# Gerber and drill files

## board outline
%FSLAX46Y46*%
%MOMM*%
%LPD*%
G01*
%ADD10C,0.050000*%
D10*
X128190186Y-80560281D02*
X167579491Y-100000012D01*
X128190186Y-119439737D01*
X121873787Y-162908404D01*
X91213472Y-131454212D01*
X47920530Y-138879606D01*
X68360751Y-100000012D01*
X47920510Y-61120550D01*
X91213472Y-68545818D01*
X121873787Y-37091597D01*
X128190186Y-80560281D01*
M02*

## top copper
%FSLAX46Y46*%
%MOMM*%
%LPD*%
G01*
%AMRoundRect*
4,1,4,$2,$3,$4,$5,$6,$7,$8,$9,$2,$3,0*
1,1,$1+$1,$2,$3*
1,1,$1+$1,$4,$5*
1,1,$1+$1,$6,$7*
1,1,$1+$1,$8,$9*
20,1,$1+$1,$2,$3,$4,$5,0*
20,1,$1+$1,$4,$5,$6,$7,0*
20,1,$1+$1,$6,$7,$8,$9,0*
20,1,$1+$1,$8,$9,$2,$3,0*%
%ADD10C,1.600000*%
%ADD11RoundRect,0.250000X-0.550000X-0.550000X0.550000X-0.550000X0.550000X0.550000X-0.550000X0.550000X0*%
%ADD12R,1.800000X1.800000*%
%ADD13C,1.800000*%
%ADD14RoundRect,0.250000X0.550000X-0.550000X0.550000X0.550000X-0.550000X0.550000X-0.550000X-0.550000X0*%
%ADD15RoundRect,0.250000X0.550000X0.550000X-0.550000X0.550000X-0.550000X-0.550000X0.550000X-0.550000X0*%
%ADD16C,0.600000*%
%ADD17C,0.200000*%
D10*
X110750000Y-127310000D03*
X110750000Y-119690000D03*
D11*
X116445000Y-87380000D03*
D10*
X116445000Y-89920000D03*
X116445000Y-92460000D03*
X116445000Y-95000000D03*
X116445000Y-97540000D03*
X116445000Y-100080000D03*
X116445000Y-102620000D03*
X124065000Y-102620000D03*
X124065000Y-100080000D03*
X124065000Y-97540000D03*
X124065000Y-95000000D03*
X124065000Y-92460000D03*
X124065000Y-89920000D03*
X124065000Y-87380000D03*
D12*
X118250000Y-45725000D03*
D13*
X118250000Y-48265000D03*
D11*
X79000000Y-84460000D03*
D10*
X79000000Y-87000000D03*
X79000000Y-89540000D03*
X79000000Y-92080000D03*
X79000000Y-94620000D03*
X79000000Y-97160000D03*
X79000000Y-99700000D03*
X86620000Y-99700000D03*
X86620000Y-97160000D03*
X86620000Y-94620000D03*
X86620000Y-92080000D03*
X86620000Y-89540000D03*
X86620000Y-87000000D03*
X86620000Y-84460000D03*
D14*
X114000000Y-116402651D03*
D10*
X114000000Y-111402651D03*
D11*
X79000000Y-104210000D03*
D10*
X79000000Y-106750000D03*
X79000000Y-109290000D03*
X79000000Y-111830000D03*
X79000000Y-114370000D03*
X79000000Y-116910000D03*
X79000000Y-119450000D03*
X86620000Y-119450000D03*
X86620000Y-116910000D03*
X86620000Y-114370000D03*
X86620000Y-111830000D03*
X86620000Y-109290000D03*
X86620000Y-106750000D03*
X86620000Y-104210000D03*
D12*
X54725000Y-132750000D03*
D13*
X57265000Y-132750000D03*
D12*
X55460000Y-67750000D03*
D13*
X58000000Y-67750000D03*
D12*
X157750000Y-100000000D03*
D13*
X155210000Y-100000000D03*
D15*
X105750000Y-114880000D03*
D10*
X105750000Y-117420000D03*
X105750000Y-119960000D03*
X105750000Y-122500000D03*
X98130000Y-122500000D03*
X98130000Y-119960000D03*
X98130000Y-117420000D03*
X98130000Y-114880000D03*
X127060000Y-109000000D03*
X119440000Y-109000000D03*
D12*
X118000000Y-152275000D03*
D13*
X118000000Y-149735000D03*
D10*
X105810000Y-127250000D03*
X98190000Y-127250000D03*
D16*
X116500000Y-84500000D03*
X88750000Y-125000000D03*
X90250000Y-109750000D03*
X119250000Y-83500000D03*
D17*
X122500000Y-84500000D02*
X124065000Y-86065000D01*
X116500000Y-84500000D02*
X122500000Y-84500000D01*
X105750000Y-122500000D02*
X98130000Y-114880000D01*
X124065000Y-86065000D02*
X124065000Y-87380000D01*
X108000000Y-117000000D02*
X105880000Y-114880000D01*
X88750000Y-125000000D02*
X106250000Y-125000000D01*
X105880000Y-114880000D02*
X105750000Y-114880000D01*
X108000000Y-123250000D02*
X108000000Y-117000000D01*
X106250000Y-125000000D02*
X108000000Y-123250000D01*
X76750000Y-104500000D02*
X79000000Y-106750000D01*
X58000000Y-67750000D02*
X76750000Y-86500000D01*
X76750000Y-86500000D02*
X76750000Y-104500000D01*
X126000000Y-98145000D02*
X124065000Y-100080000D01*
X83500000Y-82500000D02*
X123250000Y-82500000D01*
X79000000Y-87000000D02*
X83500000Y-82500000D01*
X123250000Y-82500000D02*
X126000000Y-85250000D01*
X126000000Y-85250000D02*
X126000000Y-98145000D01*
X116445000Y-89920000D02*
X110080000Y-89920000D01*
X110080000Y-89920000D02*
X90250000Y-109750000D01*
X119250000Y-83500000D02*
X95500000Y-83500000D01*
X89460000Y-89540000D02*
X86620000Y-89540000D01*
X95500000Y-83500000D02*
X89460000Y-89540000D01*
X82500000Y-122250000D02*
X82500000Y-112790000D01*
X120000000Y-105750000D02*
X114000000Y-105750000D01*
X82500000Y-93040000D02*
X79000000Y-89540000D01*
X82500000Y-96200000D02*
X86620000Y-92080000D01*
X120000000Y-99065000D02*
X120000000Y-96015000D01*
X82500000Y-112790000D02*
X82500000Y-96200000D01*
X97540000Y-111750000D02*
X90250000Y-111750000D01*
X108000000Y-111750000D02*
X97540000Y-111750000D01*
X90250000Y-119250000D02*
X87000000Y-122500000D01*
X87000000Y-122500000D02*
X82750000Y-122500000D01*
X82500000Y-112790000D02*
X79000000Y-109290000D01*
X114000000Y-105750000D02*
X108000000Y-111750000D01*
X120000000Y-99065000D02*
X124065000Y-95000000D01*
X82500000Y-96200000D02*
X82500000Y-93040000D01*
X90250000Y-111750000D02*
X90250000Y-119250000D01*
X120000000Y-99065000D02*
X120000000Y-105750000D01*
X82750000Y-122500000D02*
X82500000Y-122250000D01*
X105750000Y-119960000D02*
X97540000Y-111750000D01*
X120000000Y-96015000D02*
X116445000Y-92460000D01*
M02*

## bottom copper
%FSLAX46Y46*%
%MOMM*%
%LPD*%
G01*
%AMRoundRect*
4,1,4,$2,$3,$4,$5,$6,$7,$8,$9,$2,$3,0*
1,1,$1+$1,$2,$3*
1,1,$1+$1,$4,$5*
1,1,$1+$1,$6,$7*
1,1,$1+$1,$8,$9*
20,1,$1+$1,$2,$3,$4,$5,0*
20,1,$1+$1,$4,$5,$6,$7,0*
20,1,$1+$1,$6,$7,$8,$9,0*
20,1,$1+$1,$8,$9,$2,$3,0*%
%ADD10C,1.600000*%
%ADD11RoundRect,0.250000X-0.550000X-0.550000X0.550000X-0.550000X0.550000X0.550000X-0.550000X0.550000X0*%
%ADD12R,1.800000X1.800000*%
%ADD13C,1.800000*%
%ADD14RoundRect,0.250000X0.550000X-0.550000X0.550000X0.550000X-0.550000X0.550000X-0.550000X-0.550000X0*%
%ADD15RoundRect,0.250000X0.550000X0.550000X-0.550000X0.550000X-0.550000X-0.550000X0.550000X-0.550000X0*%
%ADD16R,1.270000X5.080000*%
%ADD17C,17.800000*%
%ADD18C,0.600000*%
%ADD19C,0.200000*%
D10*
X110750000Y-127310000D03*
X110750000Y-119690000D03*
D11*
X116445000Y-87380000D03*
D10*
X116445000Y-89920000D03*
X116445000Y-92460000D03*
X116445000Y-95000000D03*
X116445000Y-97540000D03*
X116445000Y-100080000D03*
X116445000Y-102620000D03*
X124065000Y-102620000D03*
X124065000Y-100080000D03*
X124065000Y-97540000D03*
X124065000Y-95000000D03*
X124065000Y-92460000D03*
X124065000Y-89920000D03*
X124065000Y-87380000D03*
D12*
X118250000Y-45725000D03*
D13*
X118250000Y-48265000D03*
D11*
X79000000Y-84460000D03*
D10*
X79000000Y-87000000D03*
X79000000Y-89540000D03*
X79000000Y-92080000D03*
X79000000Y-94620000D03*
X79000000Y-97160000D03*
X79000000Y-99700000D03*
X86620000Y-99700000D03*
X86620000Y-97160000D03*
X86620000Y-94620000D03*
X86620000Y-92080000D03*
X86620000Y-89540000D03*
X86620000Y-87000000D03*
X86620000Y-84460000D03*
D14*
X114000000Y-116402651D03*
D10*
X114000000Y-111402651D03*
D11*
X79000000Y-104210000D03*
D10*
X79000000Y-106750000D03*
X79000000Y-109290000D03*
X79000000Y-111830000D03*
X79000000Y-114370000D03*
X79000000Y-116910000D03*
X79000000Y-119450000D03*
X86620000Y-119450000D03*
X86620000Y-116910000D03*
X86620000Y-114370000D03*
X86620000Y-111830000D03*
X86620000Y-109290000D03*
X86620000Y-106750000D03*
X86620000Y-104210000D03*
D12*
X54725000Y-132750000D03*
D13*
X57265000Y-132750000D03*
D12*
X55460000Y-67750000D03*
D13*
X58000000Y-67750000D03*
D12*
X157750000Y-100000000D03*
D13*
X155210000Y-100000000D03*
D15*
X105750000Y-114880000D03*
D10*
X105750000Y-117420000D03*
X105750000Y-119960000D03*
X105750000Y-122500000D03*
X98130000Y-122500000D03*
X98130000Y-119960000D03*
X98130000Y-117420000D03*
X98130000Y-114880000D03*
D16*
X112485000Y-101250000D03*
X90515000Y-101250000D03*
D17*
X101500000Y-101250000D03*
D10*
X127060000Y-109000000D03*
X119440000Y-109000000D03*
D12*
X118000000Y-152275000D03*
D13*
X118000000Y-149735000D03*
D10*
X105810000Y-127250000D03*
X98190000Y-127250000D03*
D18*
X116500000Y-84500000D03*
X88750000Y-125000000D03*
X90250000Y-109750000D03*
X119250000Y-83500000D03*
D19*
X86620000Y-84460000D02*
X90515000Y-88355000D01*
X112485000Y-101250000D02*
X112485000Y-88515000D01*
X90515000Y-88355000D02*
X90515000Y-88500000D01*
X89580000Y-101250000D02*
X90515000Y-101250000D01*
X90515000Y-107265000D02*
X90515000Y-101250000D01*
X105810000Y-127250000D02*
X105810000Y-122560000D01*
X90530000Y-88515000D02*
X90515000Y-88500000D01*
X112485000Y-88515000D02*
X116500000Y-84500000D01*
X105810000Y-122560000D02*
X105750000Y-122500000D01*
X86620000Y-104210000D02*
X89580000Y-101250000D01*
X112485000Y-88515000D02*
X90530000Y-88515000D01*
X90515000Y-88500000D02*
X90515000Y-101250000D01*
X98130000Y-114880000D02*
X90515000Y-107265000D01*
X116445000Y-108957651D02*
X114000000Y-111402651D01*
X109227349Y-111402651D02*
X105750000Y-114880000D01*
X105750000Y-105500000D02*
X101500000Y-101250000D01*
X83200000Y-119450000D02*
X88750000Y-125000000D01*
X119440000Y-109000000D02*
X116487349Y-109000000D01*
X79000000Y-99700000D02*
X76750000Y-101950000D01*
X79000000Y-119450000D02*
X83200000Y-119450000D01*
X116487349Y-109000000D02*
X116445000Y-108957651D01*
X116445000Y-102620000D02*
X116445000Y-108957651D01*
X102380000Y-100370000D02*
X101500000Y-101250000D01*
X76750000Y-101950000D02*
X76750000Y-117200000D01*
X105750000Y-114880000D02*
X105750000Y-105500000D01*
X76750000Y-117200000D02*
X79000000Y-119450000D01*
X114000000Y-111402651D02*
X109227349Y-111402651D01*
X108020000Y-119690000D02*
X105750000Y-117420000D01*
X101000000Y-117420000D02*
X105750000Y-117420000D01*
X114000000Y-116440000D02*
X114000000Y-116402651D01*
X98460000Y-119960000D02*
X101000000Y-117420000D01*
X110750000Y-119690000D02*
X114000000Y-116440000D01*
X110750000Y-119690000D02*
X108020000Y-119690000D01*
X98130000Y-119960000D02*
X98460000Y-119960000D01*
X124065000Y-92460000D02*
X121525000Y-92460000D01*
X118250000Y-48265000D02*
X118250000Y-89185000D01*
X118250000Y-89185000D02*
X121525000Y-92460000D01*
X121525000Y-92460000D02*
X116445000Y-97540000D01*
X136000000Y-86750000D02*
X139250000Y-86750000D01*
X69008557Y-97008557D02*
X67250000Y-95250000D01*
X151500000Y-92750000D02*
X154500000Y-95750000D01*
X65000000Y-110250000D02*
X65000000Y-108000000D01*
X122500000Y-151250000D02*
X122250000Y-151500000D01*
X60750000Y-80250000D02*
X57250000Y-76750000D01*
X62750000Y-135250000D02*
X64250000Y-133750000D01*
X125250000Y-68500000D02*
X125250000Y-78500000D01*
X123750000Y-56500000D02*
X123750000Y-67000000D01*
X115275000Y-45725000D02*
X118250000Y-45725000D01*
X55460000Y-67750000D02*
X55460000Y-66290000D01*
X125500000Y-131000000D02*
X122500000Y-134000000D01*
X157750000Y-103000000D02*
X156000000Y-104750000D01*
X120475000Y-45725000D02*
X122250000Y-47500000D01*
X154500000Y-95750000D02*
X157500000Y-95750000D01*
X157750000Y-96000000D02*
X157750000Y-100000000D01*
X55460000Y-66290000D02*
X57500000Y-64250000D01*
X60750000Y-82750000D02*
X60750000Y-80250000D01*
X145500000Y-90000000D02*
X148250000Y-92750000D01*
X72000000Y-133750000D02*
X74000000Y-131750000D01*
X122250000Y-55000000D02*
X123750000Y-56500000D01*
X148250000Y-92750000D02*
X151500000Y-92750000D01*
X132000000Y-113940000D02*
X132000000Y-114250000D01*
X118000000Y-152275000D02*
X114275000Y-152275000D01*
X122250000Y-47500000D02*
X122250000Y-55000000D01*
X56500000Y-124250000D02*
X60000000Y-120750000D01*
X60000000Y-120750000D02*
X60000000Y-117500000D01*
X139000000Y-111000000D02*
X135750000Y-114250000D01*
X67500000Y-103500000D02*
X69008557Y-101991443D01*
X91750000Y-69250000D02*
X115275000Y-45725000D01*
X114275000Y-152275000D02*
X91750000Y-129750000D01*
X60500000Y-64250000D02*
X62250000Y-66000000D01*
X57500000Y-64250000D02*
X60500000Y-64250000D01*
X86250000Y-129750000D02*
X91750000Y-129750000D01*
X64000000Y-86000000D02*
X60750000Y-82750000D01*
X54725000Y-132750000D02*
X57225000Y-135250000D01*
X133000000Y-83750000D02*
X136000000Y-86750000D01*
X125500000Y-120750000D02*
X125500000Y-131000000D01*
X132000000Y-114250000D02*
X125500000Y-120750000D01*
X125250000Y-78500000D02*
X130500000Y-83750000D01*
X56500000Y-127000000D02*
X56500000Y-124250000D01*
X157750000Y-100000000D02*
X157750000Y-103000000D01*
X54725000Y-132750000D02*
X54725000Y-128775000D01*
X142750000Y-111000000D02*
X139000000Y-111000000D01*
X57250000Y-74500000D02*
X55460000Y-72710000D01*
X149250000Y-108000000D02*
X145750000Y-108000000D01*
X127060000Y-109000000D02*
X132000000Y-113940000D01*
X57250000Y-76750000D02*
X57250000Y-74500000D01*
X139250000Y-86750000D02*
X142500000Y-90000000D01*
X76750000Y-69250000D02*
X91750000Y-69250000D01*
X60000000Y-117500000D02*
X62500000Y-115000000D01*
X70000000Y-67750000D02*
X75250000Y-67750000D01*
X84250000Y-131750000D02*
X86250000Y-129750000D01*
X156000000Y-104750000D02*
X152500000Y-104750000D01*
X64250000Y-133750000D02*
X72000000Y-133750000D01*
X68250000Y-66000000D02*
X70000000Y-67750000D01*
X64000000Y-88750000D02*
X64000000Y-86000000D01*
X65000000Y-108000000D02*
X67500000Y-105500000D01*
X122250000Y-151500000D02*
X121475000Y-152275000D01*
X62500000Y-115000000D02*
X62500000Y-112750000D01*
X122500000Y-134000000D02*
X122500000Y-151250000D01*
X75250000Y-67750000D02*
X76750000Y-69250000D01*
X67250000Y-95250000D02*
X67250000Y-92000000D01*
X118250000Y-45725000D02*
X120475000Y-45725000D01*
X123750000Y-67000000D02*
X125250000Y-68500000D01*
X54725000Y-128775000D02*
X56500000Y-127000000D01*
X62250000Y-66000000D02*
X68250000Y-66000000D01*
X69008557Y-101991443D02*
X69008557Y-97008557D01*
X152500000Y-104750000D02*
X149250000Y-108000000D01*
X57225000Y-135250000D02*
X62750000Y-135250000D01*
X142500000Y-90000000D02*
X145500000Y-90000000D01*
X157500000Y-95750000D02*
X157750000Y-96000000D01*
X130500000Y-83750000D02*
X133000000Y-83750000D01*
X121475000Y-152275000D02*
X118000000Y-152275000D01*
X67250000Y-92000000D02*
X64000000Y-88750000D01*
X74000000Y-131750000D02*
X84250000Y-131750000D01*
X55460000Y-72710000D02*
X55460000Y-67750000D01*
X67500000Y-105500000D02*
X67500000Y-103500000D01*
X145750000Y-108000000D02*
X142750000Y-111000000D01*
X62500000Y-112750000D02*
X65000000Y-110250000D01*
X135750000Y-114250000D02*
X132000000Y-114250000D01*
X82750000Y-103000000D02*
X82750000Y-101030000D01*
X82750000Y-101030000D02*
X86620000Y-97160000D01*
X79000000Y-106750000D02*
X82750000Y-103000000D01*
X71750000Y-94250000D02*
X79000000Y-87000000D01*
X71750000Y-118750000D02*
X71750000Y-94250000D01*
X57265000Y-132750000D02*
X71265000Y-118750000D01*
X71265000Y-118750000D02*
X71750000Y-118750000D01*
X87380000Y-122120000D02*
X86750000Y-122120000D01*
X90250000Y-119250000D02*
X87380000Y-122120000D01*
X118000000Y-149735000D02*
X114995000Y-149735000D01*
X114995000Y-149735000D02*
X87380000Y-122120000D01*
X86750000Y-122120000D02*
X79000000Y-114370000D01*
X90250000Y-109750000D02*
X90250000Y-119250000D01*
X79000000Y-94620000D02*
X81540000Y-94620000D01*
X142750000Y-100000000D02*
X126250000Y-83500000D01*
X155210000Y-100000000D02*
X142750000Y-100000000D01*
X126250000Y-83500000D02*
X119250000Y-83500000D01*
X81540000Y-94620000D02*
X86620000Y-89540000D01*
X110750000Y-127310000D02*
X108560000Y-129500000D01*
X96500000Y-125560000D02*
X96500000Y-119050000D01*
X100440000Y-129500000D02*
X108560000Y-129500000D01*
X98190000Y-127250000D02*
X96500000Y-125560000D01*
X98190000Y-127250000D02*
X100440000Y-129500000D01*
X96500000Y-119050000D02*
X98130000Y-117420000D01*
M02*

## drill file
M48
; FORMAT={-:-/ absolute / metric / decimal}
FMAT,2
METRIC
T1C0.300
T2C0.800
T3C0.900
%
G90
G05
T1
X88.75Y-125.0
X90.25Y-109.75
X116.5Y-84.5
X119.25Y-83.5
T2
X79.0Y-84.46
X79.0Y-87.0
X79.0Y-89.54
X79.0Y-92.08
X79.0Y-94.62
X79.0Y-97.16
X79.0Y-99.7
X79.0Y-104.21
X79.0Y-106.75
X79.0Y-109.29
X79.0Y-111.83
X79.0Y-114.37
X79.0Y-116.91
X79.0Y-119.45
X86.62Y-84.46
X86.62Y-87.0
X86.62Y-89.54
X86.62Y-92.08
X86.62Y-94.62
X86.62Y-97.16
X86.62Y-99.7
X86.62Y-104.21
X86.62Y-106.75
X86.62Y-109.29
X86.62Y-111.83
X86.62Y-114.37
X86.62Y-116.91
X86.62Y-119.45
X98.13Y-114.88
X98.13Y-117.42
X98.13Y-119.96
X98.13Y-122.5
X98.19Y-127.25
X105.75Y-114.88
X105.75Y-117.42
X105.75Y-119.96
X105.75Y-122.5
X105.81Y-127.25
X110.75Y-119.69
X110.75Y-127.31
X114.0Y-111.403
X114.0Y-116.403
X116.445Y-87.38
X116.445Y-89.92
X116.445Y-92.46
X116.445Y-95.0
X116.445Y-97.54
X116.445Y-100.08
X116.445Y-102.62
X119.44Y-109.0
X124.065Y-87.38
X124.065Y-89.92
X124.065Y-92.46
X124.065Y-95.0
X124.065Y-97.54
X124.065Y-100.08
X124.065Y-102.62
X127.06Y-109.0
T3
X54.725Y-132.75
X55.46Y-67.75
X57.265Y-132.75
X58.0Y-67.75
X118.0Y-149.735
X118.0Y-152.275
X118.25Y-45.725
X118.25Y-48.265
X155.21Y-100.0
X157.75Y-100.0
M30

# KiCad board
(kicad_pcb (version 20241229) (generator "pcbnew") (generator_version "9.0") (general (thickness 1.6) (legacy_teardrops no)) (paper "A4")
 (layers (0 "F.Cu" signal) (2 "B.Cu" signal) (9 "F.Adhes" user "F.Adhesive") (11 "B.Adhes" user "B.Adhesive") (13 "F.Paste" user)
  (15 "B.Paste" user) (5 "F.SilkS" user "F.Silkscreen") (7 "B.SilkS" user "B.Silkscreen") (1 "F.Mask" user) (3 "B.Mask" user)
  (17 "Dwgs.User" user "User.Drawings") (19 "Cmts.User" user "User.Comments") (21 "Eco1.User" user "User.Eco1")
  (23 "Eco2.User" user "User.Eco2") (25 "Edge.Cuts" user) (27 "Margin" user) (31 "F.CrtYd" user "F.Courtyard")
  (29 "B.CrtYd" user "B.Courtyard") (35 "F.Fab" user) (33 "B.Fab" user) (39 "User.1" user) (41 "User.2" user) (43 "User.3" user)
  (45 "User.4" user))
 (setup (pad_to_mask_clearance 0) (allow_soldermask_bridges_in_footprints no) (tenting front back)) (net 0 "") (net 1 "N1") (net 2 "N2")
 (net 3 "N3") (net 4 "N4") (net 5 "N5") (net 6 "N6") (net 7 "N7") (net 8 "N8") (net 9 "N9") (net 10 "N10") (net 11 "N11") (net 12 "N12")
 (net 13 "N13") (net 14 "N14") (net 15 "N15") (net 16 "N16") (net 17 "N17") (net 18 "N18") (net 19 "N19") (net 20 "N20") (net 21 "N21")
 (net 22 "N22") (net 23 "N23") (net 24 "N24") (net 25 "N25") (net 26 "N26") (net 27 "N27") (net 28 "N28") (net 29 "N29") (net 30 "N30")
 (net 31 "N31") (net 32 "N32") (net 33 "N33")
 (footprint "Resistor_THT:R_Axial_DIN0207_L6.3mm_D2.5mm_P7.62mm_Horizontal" (layer "F.Cu") (at 110.75 127.31 90)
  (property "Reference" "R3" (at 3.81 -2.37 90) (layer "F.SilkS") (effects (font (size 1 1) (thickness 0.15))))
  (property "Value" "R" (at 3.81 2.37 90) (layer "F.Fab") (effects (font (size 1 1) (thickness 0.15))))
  (pad "1" thru_hole circle (at 0 0 90) (size 1.6 1.6) (drill 0.8) (layers "*.Cu" "*.Mask") (remove_unused_layers no) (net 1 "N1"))
  (pad "2" thru_hole circle (at 7.62 0 90) (size 1.6 1.6) (drill 0.8) (layers "*.Cu" "*.Mask") (remove_unused_layers no) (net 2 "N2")))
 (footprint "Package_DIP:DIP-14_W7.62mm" (layer "F.Cu") (at 116.445 87.38)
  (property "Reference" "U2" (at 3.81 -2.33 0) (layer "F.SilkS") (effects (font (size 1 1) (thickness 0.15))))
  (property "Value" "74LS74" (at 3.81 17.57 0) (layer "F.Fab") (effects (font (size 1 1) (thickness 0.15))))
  (pad "1" thru_hole roundrect (at 0 0) (size 1.6 1.6) (drill 0.8) (layers "*.Cu" "*.Mask") (remove_unused_layers no)
   (roundrect_rratio 0.15625) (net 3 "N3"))
  (pad "2" thru_hole circle (at 0 2.54) (size 1.6 1.6) (drill 0.8) (layers "*.Cu" "*.Mask") (remove_unused_layers no) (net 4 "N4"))
  (pad "3" thru_hole circle (at 0 5.08) (size 1.6 1.6) (drill 0.8) (layers "*.Cu" "*.Mask") (remove_unused_layers no) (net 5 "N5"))
  (pad "4" thru_hole circle (at 0 7.62) (size 1.6 1.6) (drill 0.8) (layers "*.Cu" "*.Mask") (remove_unused_layers no) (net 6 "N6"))
  (pad "5" thru_hole circle (at 0 10.16) (size 1.6 1.6) (drill 0.8) (layers "*.Cu" "*.Mask") (remove_unused_layers no) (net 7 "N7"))
  (pad "6" thru_hole circle (at 0 12.7) (size 1.6 1.6) (drill 0.8) (layers "*.Cu" "*.Mask") (remove_unused_layers no) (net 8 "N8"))
  (pad "7" thru_hole circle (at 0 15.24) (size 1.6 1.6) (drill 0.8) (layers "*.Cu" "*.Mask") (remove_unused_layers no) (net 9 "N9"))
  (pad "8" thru_hole circle (at 7.62 15.24) (size 1.6 1.6) (drill 0.8) (layers "*.Cu" "*.Mask") (remove_unused_layers no) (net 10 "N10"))
  (pad "9" thru_hole circle (at 7.62 12.7) (size 1.6 1.6) (drill 0.8) (layers "*.Cu" "*.Mask") (remove_unused_layers no) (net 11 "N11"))
  (pad "10" thru_hole circle (at 7.62 10.16) (size 1.6 1.6) (drill 0.8) (layers "*.Cu" "*.Mask") (remove_unused_layers no) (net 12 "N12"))
  (pad "11" thru_hole circle (at 7.62 7.62) (size 1.6 1.6) (drill 0.8) (layers "*.Cu" "*.Mask") (remove_unused_layers no) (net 5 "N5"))
  (pad "12" thru_hole circle (at 7.62 5.08) (size 1.6 1.6) (drill 0.8) (layers "*.Cu" "*.Mask") (remove_unused_layers no) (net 7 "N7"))
  (pad "13" thru_hole circle (at 7.62 2.54) (size 1.6 1.6) (drill 0.8) (layers "*.Cu" "*.Mask") (remove_unused_layers no) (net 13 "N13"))
  (pad "14" thru_hole circle (at 7.62 0) (size 1.6 1.6) (drill 0.8) (layers "*.Cu" "*.Mask") (remove_unused_layers no) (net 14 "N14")))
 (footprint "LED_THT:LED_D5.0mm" (layer "F.Cu") (at 118.25 45.725 -90)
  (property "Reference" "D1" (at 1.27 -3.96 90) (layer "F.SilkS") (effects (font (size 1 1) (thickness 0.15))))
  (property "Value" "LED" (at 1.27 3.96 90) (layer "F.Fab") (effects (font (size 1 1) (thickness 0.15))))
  (pad "1" thru_hole rect (at 0 0 270) (size 1.8 1.8) (drill 0.9) (layers "*.Cu" "*.Mask") (remove_unused_layers no) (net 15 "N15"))
  (pad "2" thru_hole circle (at 2.54 0 270) (size 1.8 1.8) (drill 0.9) (layers "*.Cu" "*.Mask") (remove_unused_layers no) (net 7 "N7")))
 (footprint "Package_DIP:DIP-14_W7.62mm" (layer "F.Cu") (at 79 84.46)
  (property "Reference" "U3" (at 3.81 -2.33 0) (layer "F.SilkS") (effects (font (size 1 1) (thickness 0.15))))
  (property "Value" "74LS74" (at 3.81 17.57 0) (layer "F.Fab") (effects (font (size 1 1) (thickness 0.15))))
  (pad "1" thru_hole roundrect (at 0 0) (size 1.6 1.6) (drill 0.8) (layers "*.Cu" "*.Mask") (remove_unused_layers no)
   (roundrect_rratio 0.15625) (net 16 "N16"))
  (pad "2" thru_hole circle (at 0 2.54) (size 1.6 1.6) (drill 0.8) (layers "*.Cu" "*.Mask") (remove_unused_layers no) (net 11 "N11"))
  (pad "3" thru_hole circle (at 0 5.08) (size 1.6 1.6) (drill 0.8) (layers "*.Cu" "*.Mask") (remove_unused_layers no) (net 5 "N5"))
  (pad "4" thru_hole circle (at 0 7.62) (size 1.6 1.6) (drill 0.8) (layers "*.Cu" "*.Mask") (remove_unused_layers no) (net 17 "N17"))
  (pad "5" thru_hole circle (at 0 10.16) (size 1.6 1.6) (drill 0.8) (layers "*.Cu" "*.Mask") (remove_unused_layers no) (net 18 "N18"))
  (pad "6" thru_hole circle (at 0 12.7) (size 1.6 1.6) (drill 0.8) (layers "*.Cu" "*.Mask") (remove_unused_layers no) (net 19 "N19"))
  (pad "7" thru_hole circle (at 0 15.24) (size 1.6 1.6) (drill 0.8) (layers "*.Cu" "*.Mask") (remove_unused_layers no) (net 9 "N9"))
  (pad "8" thru_hole circle (at 7.62 15.24) (size 1.6 1.6) (drill 0.8) (layers "*.Cu" "*.Mask") (remove_unused_layers no) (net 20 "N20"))
  (pad "9" thru_hole circle (at 7.62 12.7) (size 1.6 1.6) (drill 0.8) (layers "*.Cu" "*.Mask") (remove_unused_layers no) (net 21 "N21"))
  (pad "10" thru_hole circle (at 7.62 10.16) (size 1.6 1.6) (drill 0.8) (layers "*.Cu" "*.Mask") (remove_unused_layers no) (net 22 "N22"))
  (pad "11" thru_hole circle (at 7.62 7.62) (size 1.6 1.6) (drill 0.8) (layers "*.Cu" "*.Mask") (remove_unused_layers no) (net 5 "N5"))
  (pad "12" thru_hole circle (at 7.62 5.08) (size 1.6 1.6) (drill 0.8) (layers "*.Cu" "*.Mask") (remove_unused_layers no) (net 18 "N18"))
  (pad "13" thru_hole circle (at 7.62 2.54) (size 1.6 1.6) (drill 0.8) (layers "*.Cu" "*.Mask") (remove_unused_layers no) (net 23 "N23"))
  (pad "14" thru_hole circle (at 7.62 0) (size 1.6 1.6) (drill 0.8) (layers "*.Cu" "*.Mask") (remove_unused_layers no) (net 14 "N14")))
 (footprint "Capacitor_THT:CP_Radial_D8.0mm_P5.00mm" (layer "F.Cu") (at 114 116.402651 90)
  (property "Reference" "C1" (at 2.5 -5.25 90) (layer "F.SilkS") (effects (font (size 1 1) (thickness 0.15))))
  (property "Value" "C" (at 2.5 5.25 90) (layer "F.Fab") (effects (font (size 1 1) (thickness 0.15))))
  (pad "1" thru_hole roundrect (at 0 0 90) (size 1.6 1.6) (drill 0.8) (layers "*.Cu" "*.Mask") (remove_unused_layers no)
   (roundrect_rratio 0.15625) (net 2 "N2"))
  (pad "2" thru_hole circle (at 5 0 90) (size 1.6 1.6) (drill 0.8) (layers "*.Cu" "*.Mask") (remove_unused_layers no) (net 9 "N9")))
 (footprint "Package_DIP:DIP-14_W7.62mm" (layer "F.Cu") (at 79 104.21)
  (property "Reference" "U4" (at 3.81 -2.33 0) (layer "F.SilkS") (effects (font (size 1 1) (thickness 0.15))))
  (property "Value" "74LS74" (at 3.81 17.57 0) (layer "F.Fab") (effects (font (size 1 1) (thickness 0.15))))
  (pad "1" thru_hole roundrect (at 0 0) (size 1.6 1.6) (drill 0.8) (layers "*.Cu" "*.Mask") (remove_unused_layers no)
   (roundrect_rratio 0.15625) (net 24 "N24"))
  (pad "2" thru_hole circle (at 0 2.54) (size 1.6 1.6) (drill 0.8) (layers "*.Cu" "*.Mask") (remove_unused_layers no) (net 21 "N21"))
  (pad "3" thru_hole circle (at 0 5.08) (size 1.6 1.6) (drill 0.8) (layers "*.Cu" "*.Mask") (remove_unused_layers no) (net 5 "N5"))
  (pad "4" thru_hole circle (at 0 7.62) (size 1.6 1.6) (drill 0.8) (layers "*.Cu" "*.Mask") (remove_unused_layers no) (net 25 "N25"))
  (pad "5" thru_hole circle (at 0 10.16) (size 1.6 1.6) (drill 0.8) (layers "*.Cu" "*.Mask") (remove_unused_layers no) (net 4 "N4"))
  (pad "6" thru_hole circle (at 0 12.7) (size 1.6 1.6) (drill 0.8) (layers "*.Cu" "*.Mask") (remove_unused_layers no) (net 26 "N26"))
  (pad "7" thru_hole circle (at 0 15.24) (size 1.6 1.6) (drill 0.8) (layers "*.Cu" "*.Mask") (remove_unused_layers no) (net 9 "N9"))
  (pad "8" thru_hole circle (at 7.62 15.24) (size 1.6 1.6) (drill 0.8) (layers "*.Cu" "*.Mask") (remove_unused_layers no) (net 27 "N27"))
  (pad "9" thru_hole circle (at 7.62 12.7) (size 1.6 1.6) (drill 0.8) (layers "*.Cu" "*.Mask") (remove_unused_layers no) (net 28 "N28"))
  (pad "10" thru_hole circle (at 7.62 10.16) (size 1.6 1.6) (drill 0.8) (layers "*.Cu" "*.Mask") (remove_unused_layers no) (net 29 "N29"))
  (pad "11" thru_hole circle (at 7.62 7.62) (size 1.6 1.6) (drill 0.8) (layers "*.Cu" "*.Mask") (remove_unused_layers no) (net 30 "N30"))
  (pad "12" thru_hole circle (at 7.62 5.08) (size 1.6 1.6) (drill 0.8) (layers "*.Cu" "*.Mask") (remove_unused_layers no) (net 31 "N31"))
  (pad "13" thru_hole circle (at 7.62 2.54) (size 1.6 1.6) (drill 0.8) (layers "*.Cu" "*.Mask") (remove_unused_layers no) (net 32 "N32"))
  (pad "14" thru_hole circle (at 7.62 0) (size 1.6 1.6) (drill 0.8) (layers "*.Cu" "*.Mask") (remove_unused_layers no) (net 14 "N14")))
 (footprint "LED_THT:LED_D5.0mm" (layer "F.Cu") (at 54.725 132.75)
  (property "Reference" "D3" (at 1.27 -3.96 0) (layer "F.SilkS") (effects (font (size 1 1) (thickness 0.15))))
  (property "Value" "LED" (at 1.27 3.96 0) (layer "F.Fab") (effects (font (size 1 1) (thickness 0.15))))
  (pad "1" thru_hole rect (at 0 0) (size 1.8 1.8) (drill 0.9) (layers "*.Cu" "*.Mask") (remove_unused_layers no) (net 15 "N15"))
  (pad "2" thru_hole circle (at 2.54 0) (size 1.8 1.8) (drill 0.9) (layers "*.Cu" "*.Mask") (remove_unused_layers no) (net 11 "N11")))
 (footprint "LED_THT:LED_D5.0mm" (layer "F.Cu") (at 55.46 67.75)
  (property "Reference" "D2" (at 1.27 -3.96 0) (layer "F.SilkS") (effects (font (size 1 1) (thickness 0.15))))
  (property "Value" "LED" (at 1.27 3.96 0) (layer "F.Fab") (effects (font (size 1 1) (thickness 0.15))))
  (pad "1" thru_hole rect (at 0 0) (size 1.8 1.8) (drill 0.9) (layers "*.Cu" "*.Mask") (remove_unused_layers no) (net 15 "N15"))
  (pad "2" thru_hole circle (at 2.54 0) (size 1.8 1.8) (drill 0.9) (layers "*.Cu" "*.Mask") (remove_unused_layers no) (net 21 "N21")))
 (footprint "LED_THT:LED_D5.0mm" (layer "B.Cu") (at 157.75 100 180)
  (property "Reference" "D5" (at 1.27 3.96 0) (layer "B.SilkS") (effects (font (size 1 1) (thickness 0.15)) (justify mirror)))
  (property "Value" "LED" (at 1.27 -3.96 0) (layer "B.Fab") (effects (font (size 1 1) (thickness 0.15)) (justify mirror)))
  (pad "1" thru_hole rect (at 0 0 180) (size 1.8 1.8) (drill 0.9) (layers "*.Cu" "*.Mask") (remove_unused_layers no) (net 15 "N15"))
  (pad "2" thru_hole circle (at 2.54 0 180) (size 1.8 1.8) (drill 0.9) (layers "*.Cu" "*.Mask") (remove_unused_layers no) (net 18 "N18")))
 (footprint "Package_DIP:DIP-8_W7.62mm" (layer "B.Cu") (at 105.75 114.88 180)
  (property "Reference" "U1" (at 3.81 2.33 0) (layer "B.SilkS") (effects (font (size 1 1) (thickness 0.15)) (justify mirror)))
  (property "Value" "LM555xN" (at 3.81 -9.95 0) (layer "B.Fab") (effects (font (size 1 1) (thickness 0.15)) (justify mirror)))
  (pad "1" thru_hole roundrect (at 0 0 180) (size 1.6 1.6) (drill 0.8) (layers "*.Cu" "*.Mask") (remove_unused_layers no)
   (roundrect_rratio 0.15625) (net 9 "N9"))
  (pad "2" thru_hole circle (at 0 -2.54 180) (size 1.6 1.6) (drill 0.8) (layers "*.Cu" "*.Mask") (remove_unused_layers no) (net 2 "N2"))
  (pad "3" thru_hole circle (at 0 -5.08 180) (size 1.6 1.6) (drill 0.8) (layers "*.Cu" "*.Mask") (remove_unused_layers no) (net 5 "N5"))
  (pad "4" thru_hole circle (at 0 -7.62 180) (size 1.6 1.6) (drill 0.8) (layers "*.Cu" "*.Mask") (remove_unused_layers no) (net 14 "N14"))
  (pad "5" thru_hole circle (at 7.62 -7.62 180) (size 1.6 1.6) (drill 0.8) (layers "*.Cu" "*.Mask") (remove_unused_layers no) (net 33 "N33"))
  (pad "6" thru_hole circle (at 7.62 -5.08 180) (size 1.6 1.6) (drill 0.8) (layers "*.Cu" "*.Mask") (remove_unused_layers no) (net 2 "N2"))
  (pad "7" thru_hole circle (at 7.62 -2.54 180) (size 1.6 1.6) (drill 0.8) (layers "*.Cu" "*.Mask") (remove_unused_layers no) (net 1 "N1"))
  (pad "8" thru_hole circle (at 7.62 0 180) (size 1.6 1.6) (drill 0.8) (layers "*.Cu" "*.Mask") (remove_unused_layers no) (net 14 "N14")))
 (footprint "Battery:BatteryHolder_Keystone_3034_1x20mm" (layer "B.Cu") (at 101.5 101.25 180)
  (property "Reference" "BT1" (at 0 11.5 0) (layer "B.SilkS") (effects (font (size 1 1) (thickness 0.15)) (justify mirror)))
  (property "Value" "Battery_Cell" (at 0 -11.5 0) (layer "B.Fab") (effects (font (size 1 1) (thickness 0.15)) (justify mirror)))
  (pad "1" smd rect (at -10.985 0 180) (size 1.27 5.08) (layers "B.Cu" "B.Mask" "B.Paste") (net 14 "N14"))
  (pad "1" smd rect (at 10.985 0 180) (size 1.27 5.08) (layers "B.Cu" "B.Mask" "B.Paste") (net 14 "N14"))
  (pad "2" smd circle (at 0 0 180) (size 17.8 17.8) (layers "B.Cu" "B.Mask") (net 9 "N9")))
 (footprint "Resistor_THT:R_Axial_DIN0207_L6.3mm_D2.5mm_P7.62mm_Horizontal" (layer "B.Cu") (at 127.06 109 180)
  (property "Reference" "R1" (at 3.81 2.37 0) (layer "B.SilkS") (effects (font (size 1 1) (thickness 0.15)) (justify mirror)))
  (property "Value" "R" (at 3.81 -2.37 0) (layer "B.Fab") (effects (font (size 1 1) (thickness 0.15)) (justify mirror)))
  (pad "1" thru_hole circle (at 0 0 180) (size 1.6 1.6) (drill 0.8) (layers "*.Cu" "*.Mask") (remove_unused_layers no) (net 15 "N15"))
  (pad "2" thru_hole circle (at 7.62 0 180) (size 1.6 1.6) (drill 0.8) (layers "*.Cu" "*.Mask") (remove_unused_layers no) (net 9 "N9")))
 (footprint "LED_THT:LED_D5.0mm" (layer "B.Cu") (at 118 152.275 90)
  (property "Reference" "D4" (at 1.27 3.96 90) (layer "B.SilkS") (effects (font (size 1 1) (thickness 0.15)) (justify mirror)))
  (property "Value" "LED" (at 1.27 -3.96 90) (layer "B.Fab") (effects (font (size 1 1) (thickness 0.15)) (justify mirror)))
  (pad "1" thru_hole rect (at 0 0 90) (size 1.8 1.8) (drill 0.9) (layers "*.Cu" "*.Mask") (remove_unused_layers no) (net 15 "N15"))
  (pad "2" thru_hole circle (at 2.54 0 90) (size 1.8 1.8) (drill 0.9) (layers "*.Cu" "*.Mask") (remove_unused_layers no) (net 4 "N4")))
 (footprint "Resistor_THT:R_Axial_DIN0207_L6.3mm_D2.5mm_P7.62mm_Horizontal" (layer "B.Cu") (at 105.81 127.25 180)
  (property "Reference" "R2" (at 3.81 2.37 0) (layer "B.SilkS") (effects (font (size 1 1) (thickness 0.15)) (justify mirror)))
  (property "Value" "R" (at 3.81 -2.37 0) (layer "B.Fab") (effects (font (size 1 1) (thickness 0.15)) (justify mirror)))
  (pad "1" thru_hole circle (at 0 0 180) (size 1.6 1.6) (drill 0.8) (layers "*.Cu" "*.Mask") (remove_unused_layers no) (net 14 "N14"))
  (pad "2" thru_hole circle (at 7.62 0 180) (size 1.6 1.6) (drill 0.8) (layers "*.Cu" "*.Mask") (remove_unused_layers no) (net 1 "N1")))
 (gr_poly
  (pts (xy 128.190186 80.560281) (xy 167.579491 100.000012) (xy 128.190186 119.439737) (xy 121.873787 162.908404) (xy 91.213472 131.454212)
   (xy 47.92053 138.879606) (xy 68.360751 100.000012) (xy 47.92051 61.12055) (xy 91.213472 68.545818) (xy 121.873787 37.091597))
  (stroke (width 0.05) (type solid)) (fill no) (layer "Edge.Cuts"))
 (segment (start 122.5 84.5) (end 124.065 86.065) (width 0.2) (layer "F.Cu") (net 14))
 (segment (start 116.5 84.5) (end 122.5 84.5) (width 0.2) (layer "F.Cu") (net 14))
 (segment (start 105.75 122.5) (end 98.13 114.88) (width 0.2) (layer "F.Cu") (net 14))
 (segment (start 124.065 86.065) (end 124.065 87.38) (width 0.2) (layer "F.Cu") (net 14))
 (via (at 116.5 84.5) (size 0.6) (drill 0.3) (layers "F.Cu" "B.Cu") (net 14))
 (segment (start 86.62 84.46) (end 90.515 88.355) (width 0.2) (layer "B.Cu") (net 14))
 (segment (start 112.485 101.25) (end 112.485 88.515) (width 0.2) (layer "B.Cu") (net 14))
 (segment (start 90.515 88.355) (end 90.515 88.5) (width 0.2) (layer "B.Cu") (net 14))
 (segment (start 89.58 101.25) (end 90.515 101.25) (width 0.2) (layer "B.Cu") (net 14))
 (segment (start 90.515 107.265) (end 90.515 101.25) (width 0.2) (layer "B.Cu") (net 14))
 (segment (start 105.81 127.25) (end 105.81 122.56) (width 0.2) (layer "B.Cu") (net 14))
 (segment (start 90.53 88.515) (end 90.515 88.5) (width 0.2) (layer "B.Cu") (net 14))
 (segment (start 112.485 88.515) (end 116.5 84.5) (width 0.2) (layer "B.Cu") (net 14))
 (segment (start 105.81 122.56) (end 105.75 122.5) (width 0.2) (layer "B.Cu") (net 14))
 (segment (start 86.62 104.21) (end 89.58 101.25) (width 0.2) (layer "B.Cu") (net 14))
 (segment (start 112.485 88.515) (end 90.53 88.515) (width 0.2) (layer "B.Cu") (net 14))
 (segment (start 90.515 88.5) (end 90.515 101.25) (width 0.2) (layer "B.Cu") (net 14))
 (segment (start 98.13 114.88) (end 90.515 107.265) (width 0.2) (layer "B.Cu") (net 14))
 (segment (start 108 117) (end 105.88 114.88) (width 0.2) (layer "F.Cu") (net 9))
 (segment (start 88.75 125) (end 106.25 125) (width 0.2) (layer "F.Cu") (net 9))
 (segment (start 105.88 114.88) (end 105.75 114.88) (width 0.2) (layer "F.Cu") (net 9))
 (segment (start 108 123.25) (end 108 117) (width 0.2) (layer "F.Cu") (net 9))
 (segment (start 106.25 125) (end 108 123.25) (width 0.2) (layer "F.Cu") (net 9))
 (via (at 88.75 125) (size 0.6) (drill 0.3) (layers "F.Cu" "B.Cu") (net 9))
 (segment (start 116.445 108.957651) (end 114 111.402651) (width 0.2) (layer "B.Cu") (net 9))
 (segment (start 109.227349 111.402651) (end 105.75 114.88) (width 0.2) (layer "B.Cu") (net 9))
 (segment (start 105.75 105.5) (end 101.5 101.25) (width 0.2) (layer "B.Cu") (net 9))
 (segment (start 83.2 119.45) (end 88.75 125) (width 0.2) (layer "B.Cu") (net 9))
 (segment (start 119.44 109) (end 116.487349 109) (width 0.2) (layer "B.Cu") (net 9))
 (segment (start 79 99.7) (end 76.75 101.95) (width 0.2) (layer "B.Cu") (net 9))
 (segment (start 79 119.45) (end 83.2 119.45) (width 0.2) (layer "B.Cu") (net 9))
 (segment (start 116.487349 109) (end 116.445 108.957651) (width 0.2) (layer "B.Cu") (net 9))
 (segment (start 116.445 102.62) (end 116.445 108.957651) (width 0.2) (layer "B.Cu") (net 9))
 (segment (start 102.38 100.37) (end 101.5 101.25) (width 0.2) (layer "B.Cu") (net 9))
 (segment (start 76.75 101.95) (end 76.75 117.2) (width 0.2) (layer "B.Cu") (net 9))
 (segment (start 105.75 114.88) (end 105.75 105.5) (width 0.2) (layer "B.Cu") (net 9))
 (segment (start 76.75 117.2) (end 79 119.45) (width 0.2) (layer "B.Cu") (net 9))
 (segment (start 114 111.402651) (end 109.227349 111.402651) (width 0.2) (layer "B.Cu") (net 9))
 (segment (start 108.02 119.69) (end 105.75 117.42) (width 0.2) (layer "B.Cu") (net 2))
 (segment (start 101 117.42) (end 105.75 117.42) (width 0.2) (layer "B.Cu") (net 2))
 (segment (start 114 116.44) (end 114 116.402651) (width 0.2) (layer "B.Cu") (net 2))
 (segment (start 98.46 119.96) (end 101 117.42) (width 0.2) (layer "B.Cu") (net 2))
 (segment (start 110.75 119.69) (end 114 116.44) (width 0.2) (layer "B.Cu") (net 2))
 (segment (start 110.75 119.69) (end 108.02 119.69) (width 0.2) (layer "B.Cu") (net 2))
 (segment (start 98.13 119.96) (end 98.46 119.96) (width 0.2) (layer "B.Cu") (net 2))
 (segment (start 124.065 92.46) (end 121.525 92.46) (width 0.2) (layer "B.Cu") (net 7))
 (segment (start 118.25 48.265) (end 118.25 89.185) (width 0.2) (layer "B.Cu") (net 7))
 (segment (start 118.25 89.185) (end 121.525 92.46) (width 0.2) (layer "B.Cu") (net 7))
 (segment (start 121.525 92.46) (end 116.445 97.54) (width 0.2) (layer "B.Cu") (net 7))
 (segment (start 136 86.75) (end 139.25 86.75) (width 0.2) (layer "B.Cu") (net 15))
 (segment (start 69.008557 97.008557) (end 67.25 95.25) (width 0.2) (layer "B.Cu") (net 15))
 (segment (start 151.5 92.75) (end 154.5 95.75) (width 0.2) (layer "B.Cu") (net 15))
 (segment (start 65 110.25) (end 65 108) (width 0.2) (layer "B.Cu") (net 15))
 (segment (start 122.5 151.25) (end 122.25 151.5) (width 0.2) (layer "B.Cu") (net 15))
 (segment (start 60.75 80.25) (end 57.25 76.75) (width 0.2) (layer "B.Cu") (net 15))
 (segment (start 62.75 135.25) (end 64.25 133.75) (width 0.2) (layer "B.Cu") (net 15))
 (segment (start 125.25 68.5) (end 125.25 78.5) (width 0.2) (layer "B.Cu") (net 15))
 (segment (start 123.75 56.5) (end 123.75 67) (width 0.2) (layer "B.Cu") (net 15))
 (segment (start 115.275 45.725) (end 118.25 45.725) (width 0.2) (layer "B.Cu") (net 15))
 (segment (start 55.46 67.75) (end 55.46 66.29) (width 0.2) (layer "B.Cu") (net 15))
 (segment (start 125.5 131) (end 122.5 134) (width 0.2) (layer "B.Cu") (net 15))
 (segment (start 157.75 103) (end 156 104.75) (width 0.2) (layer "B.Cu") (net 15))
 (segment (start 120.475 45.725) (end 122.25 47.5) (width 0.2) (layer "B.Cu") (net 15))
 (segment (start 154.5 95.75) (end 157.5 95.75) (width 0.2) (layer "B.Cu") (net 15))
 (segment (start 157.75 96) (end 157.75 100) (width 0.2) (layer "B.Cu") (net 15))
 (segment (start 55.46 66.29) (end 57.5 64.25) (width 0.2) (layer "B.Cu") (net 15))
 (segment (start 60.75 82.75) (end 60.75 80.25) (width 0.2) (layer "B.Cu") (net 15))
 (segment (start 145.5 90) (end 148.25 92.75) (width 0.2) (layer "B.Cu") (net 15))
 (segment (start 72 133.75) (end 74 131.75) (width 0.2) (layer "B.Cu") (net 15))
 (segment (start 122.25 55) (end 123.75 56.5) (width 0.2) (layer "B.Cu") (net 15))
 (segment (start 148.25 92.75) (end 151.5 92.75) (width 0.2) (layer "B.Cu") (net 15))
 (segment (start 132 113.94) (end 132 114.25) (width 0.2) (layer "B.Cu") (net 15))
 (segment (start 118 152.275) (end 114.275 152.275) (width 0.2) (layer "B.Cu") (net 15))
 (segment (start 122.25 47.5) (end 122.25 55) (width 0.2) (layer "B.Cu") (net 15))
 (segment (start 56.5 124.25) (end 60 120.75) (width 0.2) (layer "B.Cu") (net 15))
 (segment (start 60 120.75) (end 60 117.5) (width 0.2) (layer "B.Cu") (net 15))
 (segment (start 139 111) (end 135.75 114.25) (width 0.2) (layer "B.Cu") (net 15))
 (segment (start 67.5 103.5) (end 69.008557 101.991443) (width 0.2) (layer "B.Cu") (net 15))
 (segment (start 91.75 69.25) (end 115.275 45.725) (width 0.2) (layer "B.Cu") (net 15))
 (segment (start 114.275 152.275) (end 91.75 129.75) (width 0.2) (layer "B.Cu") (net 15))
 (segment (start 60.5 64.25) (end 62.25 66) (width 0.2) (layer "B.Cu") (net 15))
 (segment (start 57.5 64.25) (end 60.5 64.25) (width 0.2) (layer "B.Cu") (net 15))
 (segment (start 86.25 129.75) (end 91.75 129.75) (width 0.2) (layer "B.Cu") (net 15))
 (segment (start 64 86) (end 60.75 82.75) (width 0.2) (layer "B.Cu") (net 15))
 (segment (start 54.725 132.75) (end 57.225 135.25) (width 0.2) (layer "B.Cu") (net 15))
 (segment (start 133 83.75) (end 136 86.75) (width 0.2) (layer "B.Cu") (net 15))
 (segment (start 125.5 120.75) (end 125.5 131) (width 0.2) (layer "B.Cu") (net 15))
 (segment (start 132 114.25) (end 125.5 120.75) (width 0.2) (layer "B.Cu") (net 15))
 (segment (start 125.25 78.5) (end 130.5 83.75) (width 0.2) (layer "B.Cu") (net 15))
 (segment (start 56.5 127) (end 56.5 124.25) (width 0.2) (layer "B.Cu") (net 15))
 (segment (start 157.75 100) (end 157.75 103) (width 0.2) (layer "B.Cu") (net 15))
 (segment (start 54.725 132.75) (end 54.725 128.775) (width 0.2) (layer "B.Cu") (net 15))
 (segment (start 142.75 111) (end 139 111) (width 0.2) (layer "B.Cu") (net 15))
 (segment (start 57.25 74.5) (end 55.46 72.71) (width 0.2) (layer "B.Cu") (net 15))
 (segment (start 149.25 108) (end 145.75 108) (width 0.2) (layer "B.Cu") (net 15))
 (segment (start 127.06 109) (end 132 113.94) (width 0.2) (layer "B.Cu") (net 15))
 (segment (start 57.25 76.75) (end 57.25 74.5) (width 0.2) (layer "B.Cu") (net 15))
 (segment (start 139.25 86.75) (end 142.5 90) (width 0.2) (layer "B.Cu") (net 15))
 (segment (start 76.75 69.25) (end 91.75 69.25) (width 0.2) (layer "B.Cu") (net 15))
 (segment (start 60 117.5) (end 62.5 115) (width 0.2) (layer "B.Cu") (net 15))
 (segment (start 70 67.75) (end 75.25 67.75) (width 0.2) (layer "B.Cu") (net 15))
 (segment (start 84.25 131.75) (end 86.25 129.75) (width 0.2) (layer "B.Cu") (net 15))
 (segment (start 156 104.75) (end 152.5 104.75) (width 0.2) (layer "B.Cu") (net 15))
 (segment (start 64.25 133.75) (end 72 133.75) (width 0.2) (layer "B.Cu") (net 15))
 (segment (start 68.25 66) (end 70 67.75) (width 0.2) (layer "B.Cu") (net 15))
 (segment (start 64 88.75) (end 64 86) (width 0.2) (layer "B.Cu") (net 15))
 (segment (start 65 108) (end 67.5 105.5) (width 0.2) (layer "B.Cu") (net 15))
 (segment (start 122.25 151.5) (end 121.475 152.275) (width 0.2) (layer "B.Cu") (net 15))
 (segment (start 62.5 115) (end 62.5 112.75) (width 0.2) (layer "B.Cu") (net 15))
 (segment (start 122.5 134) (end 122.5 151.25) (width 0.2) (layer "B.Cu") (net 15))
 (segment (start 75.25 67.75) (end 76.75 69.25) (width 0.2) (layer "B.Cu") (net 15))
 (segment (start 67.25 95.25) (end 67.25 92) (width 0.2) (layer "B.Cu") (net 15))
 (segment (start 118.25 45.725) (end 120.475 45.725) (width 0.2) (layer "B.Cu") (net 15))
 (segment (start 123.75 67) (end 125.25 68.5) (width 0.2) (layer "B.Cu") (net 15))
 (segment (start 54.725 128.775) (end 56.5 127) (width 0.2) (layer "B.Cu") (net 15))
 (segment (start 62.25 66) (end 68.25 66) (width 0.2) (layer "B.Cu") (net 15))
 (segment (start 69.008557 101.991443) (end 69.008557 97.008557) (width 0.2) (layer "B.Cu") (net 15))
 (segment (start 152.5 104.75) (end 149.25 108) (width 0.2) (layer "B.Cu") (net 15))
 (segment (start 57.225 135.25) (end 62.75 135.25) (width 0.2) (layer "B.Cu") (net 15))
 (segment (start 142.5 90) (end 145.5 90) (width 0.2) (layer "B.Cu") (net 15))
 (segment (start 157.5 95.75) (end 157.75 96) (width 0.2) (layer "B.Cu") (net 15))
 (segment (start 130.5 83.75) (end 133 83.75) (width 0.2) (layer "B.Cu") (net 15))
 (segment (start 121.475 152.275) (end 118 152.275) (width 0.2) (layer "B.Cu") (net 15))
 (segment (start 67.25 92) (end 64 88.75) (width 0.2) (layer "B.Cu") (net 15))
 (segment (start 74 131.75) (end 84.25 131.75) (width 0.2) (layer "B.Cu") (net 15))
 (segment (start 55.46 72.71) (end 55.46 67.75) (width 0.2) (layer "B.Cu") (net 15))
 (segment (start 67.5 105.5) (end 67.5 103.5) (width 0.2) (layer "B.Cu") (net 15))
 (segment (start 145.75 108) (end 142.75 111) (width 0.2) (layer "B.Cu") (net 15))
 (segment (start 62.5 112.75) (end 65 110.25) (width 0.2) (layer "B.Cu") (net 15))
 (segment (start 135.75 114.25) (end 132 114.25) (width 0.2) (layer "B.Cu") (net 15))
 (segment (start 76.75 104.5) (end 79 106.75) (width 0.2) (layer "F.Cu") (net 21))
 (segment (start 58 67.75) (end 76.75 86.5) (width 0.2) (layer "F.Cu") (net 21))
 (segment (start 76.75 86.5) (end 76.75 104.5) (width 0.2) (layer "F.Cu") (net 21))
 (segment (start 82.75 103) (end 82.75 101.03) (width 0.2) (layer "B.Cu") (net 21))
 (segment (start 82.75 101.03) (end 86.62 97.16) (width 0.2) (layer "B.Cu") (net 21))
 (segment (start 79 106.75) (end 82.75 103) (width 0.2) (layer "B.Cu") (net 21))
 (segment (start 126 98.145) (end 124.065 100.08) (width 0.2) (layer "F.Cu") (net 11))
 (segment (start 83.5 82.5) (end 123.25 82.5) (width 0.2) (layer "F.Cu") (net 11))
 (segment (start 79 87) (end 83.5 82.5) (width 0.2) (layer "F.Cu") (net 11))
 (segment (start 123.25 82.5) (end 126 85.25) (width 0.2) (layer "F.Cu") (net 11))
 (segment (start 126 85.25) (end 126 98.145) (width 0.2) (layer "F.Cu") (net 11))
 (segment (start 71.75 94.25) (end 79 87) (width 0.2) (layer "B.Cu") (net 11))
 (segment (start 71.75 118.75) (end 71.75 94.25) (width 0.2) (layer "B.Cu") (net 11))
 (segment (start 57.265 132.75) (end 71.265 118.75) (width 0.2) (layer "B.Cu") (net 11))
 (segment (start 71.265 118.75) (end 71.75 118.75) (width 0.2) (layer "B.Cu") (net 11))
 (segment (start 116.445 89.92) (end 110.08 89.92) (width 0.2) (layer "F.Cu") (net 4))
 (segment (start 110.08 89.92) (end 90.25 109.75) (width 0.2) (layer "F.Cu") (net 4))
 (via (at 90.25 109.75) (size 0.6) (drill 0.3) (layers "F.Cu" "B.Cu") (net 4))
 (segment (start 87.38 122.12) (end 86.75 122.12) (width 0.2) (layer "B.Cu") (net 4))
 (segment (start 90.25 119.25) (end 87.38 122.12) (width 0.2) (layer "B.Cu") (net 4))
 (segment (start 118 149.735) (end 114.995 149.735) (width 0.2) (layer "B.Cu") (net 4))
 (segment (start 114.995 149.735) (end 87.38 122.12) (width 0.2) (layer "B.Cu") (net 4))
 (segment (start 86.75 122.12) (end 79 114.37) (width 0.2) (layer "B.Cu") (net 4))
 (segment (start 90.25 109.75) (end 90.25 119.25) (width 0.2) (layer "B.Cu") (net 4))
 (segment (start 119.25 83.5) (end 95.5 83.5) (width 0.2) (layer "F.Cu") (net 18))
 (segment (start 89.46 89.54) (end 86.62 89.54) (width 0.2) (layer "F.Cu") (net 18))
 (segment (start 95.5 83.5) (end 89.46 89.54) (width 0.2) (layer "F.Cu") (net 18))
 (via (at 119.25 83.5) (size 0.6) (drill 0.3) (layers "F.Cu" "B.Cu") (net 18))
 (segment (start 79 94.62) (end 81.54 94.62) (width 0.2) (layer "B.Cu") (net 18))
 (segment (start 142.75 100) (end 126.25 83.5) (width 0.2) (layer "B.Cu") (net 18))
 (segment (start 155.21 100) (end 142.75 100) (width 0.2) (layer "B.Cu") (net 18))
 (segment (start 126.25 83.5) (end 119.25 83.5) (width 0.2) (layer "B.Cu") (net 18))
 (segment (start 81.54 94.62) (end 86.62 89.54) (width 0.2) (layer "B.Cu") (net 18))
 (segment (start 110.75 127.31) (end 108.56 129.5) (width 0.2) (layer "B.Cu") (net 1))
 (segment (start 96.5 125.56) (end 96.5 119.05) (width 0.2) (layer "B.Cu") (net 1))
 (segment (start 100.44 129.5) (end 108.56 129.5) (width 0.2) (layer "B.Cu") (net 1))
 (segment (start 98.19 127.25) (end 96.5 125.56) (width 0.2) (layer "B.Cu") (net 1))
 (segment (start 98.19 127.25) (end 100.44 129.5) (width 0.2) (layer "B.Cu") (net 1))
 (segment (start 96.5 119.05) (end 98.13 117.42) (width 0.2) (layer "B.Cu") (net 1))
 (segment (start 82.5 122.25) (end 82.5 112.79) (width 0.2) (layer "F.Cu") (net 5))
 (segment (start 120 105.75) (end 114 105.75) (width 0.2) (layer "F.Cu") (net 5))
 (segment (start 82.5 93.04) (end 79 89.54) (width 0.2) (layer "F.Cu") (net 5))
 (segment (start 82.5 96.2) (end 86.62 92.08) (width 0.2) (layer "F.Cu") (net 5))
 (segment (start 120 99.065) (end 120 96.015) (width 0.2) (layer "F.Cu") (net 5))
 (segment (start 82.5 112.79) (end 82.5 96.2) (width 0.2) (layer "F.Cu") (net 5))
 (segment (start 97.54 111.75) (end 90.25 111.75) (width 0.2) (layer "F.Cu") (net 5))
 (segment (start 108 111.75) (end 97.54 111.75) (width 0.2) (layer "F.Cu") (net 5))
 (segment (start 90.25 119.25) (end 87 122.5) (width 0.2) (layer "F.Cu") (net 5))
 (segment (start 87 122.5) (end 82.75 122.5) (width 0.2) (layer "F.Cu") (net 5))
 (segment (start 82.5 112.79) (end 79 109.29) (width 0.2) (layer "F.Cu") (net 5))
 (segment (start 114 105.75) (end 108 111.75) (width 0.2) (layer "F.Cu") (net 5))
 (segment (start 120 99.065) (end 124.065 95) (width 0.2) (layer "F.Cu") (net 5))
 (segment (start 82.5 96.2) (end 82.5 93.04) (width 0.2) (layer "F.Cu") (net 5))
 (segment (start 90.25 111.75) (end 90.25 119.25) (width 0.2) (layer "F.Cu") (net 5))
 (segment (start 120 99.065) (end 120 105.75) (width 0.2) (layer "F.Cu") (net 5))
 (segment (start 82.75 122.5) (end 82.5 122.25) (width 0.2) (layer "F.Cu") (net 5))
 (segment (start 105.75 119.96) (end 97.54 111.75) (width 0.2) (layer "F.Cu") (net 5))
 (segment (start 120 96.015) (end 116.445 92.46) (width 0.2) (layer "F.Cu") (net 5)))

